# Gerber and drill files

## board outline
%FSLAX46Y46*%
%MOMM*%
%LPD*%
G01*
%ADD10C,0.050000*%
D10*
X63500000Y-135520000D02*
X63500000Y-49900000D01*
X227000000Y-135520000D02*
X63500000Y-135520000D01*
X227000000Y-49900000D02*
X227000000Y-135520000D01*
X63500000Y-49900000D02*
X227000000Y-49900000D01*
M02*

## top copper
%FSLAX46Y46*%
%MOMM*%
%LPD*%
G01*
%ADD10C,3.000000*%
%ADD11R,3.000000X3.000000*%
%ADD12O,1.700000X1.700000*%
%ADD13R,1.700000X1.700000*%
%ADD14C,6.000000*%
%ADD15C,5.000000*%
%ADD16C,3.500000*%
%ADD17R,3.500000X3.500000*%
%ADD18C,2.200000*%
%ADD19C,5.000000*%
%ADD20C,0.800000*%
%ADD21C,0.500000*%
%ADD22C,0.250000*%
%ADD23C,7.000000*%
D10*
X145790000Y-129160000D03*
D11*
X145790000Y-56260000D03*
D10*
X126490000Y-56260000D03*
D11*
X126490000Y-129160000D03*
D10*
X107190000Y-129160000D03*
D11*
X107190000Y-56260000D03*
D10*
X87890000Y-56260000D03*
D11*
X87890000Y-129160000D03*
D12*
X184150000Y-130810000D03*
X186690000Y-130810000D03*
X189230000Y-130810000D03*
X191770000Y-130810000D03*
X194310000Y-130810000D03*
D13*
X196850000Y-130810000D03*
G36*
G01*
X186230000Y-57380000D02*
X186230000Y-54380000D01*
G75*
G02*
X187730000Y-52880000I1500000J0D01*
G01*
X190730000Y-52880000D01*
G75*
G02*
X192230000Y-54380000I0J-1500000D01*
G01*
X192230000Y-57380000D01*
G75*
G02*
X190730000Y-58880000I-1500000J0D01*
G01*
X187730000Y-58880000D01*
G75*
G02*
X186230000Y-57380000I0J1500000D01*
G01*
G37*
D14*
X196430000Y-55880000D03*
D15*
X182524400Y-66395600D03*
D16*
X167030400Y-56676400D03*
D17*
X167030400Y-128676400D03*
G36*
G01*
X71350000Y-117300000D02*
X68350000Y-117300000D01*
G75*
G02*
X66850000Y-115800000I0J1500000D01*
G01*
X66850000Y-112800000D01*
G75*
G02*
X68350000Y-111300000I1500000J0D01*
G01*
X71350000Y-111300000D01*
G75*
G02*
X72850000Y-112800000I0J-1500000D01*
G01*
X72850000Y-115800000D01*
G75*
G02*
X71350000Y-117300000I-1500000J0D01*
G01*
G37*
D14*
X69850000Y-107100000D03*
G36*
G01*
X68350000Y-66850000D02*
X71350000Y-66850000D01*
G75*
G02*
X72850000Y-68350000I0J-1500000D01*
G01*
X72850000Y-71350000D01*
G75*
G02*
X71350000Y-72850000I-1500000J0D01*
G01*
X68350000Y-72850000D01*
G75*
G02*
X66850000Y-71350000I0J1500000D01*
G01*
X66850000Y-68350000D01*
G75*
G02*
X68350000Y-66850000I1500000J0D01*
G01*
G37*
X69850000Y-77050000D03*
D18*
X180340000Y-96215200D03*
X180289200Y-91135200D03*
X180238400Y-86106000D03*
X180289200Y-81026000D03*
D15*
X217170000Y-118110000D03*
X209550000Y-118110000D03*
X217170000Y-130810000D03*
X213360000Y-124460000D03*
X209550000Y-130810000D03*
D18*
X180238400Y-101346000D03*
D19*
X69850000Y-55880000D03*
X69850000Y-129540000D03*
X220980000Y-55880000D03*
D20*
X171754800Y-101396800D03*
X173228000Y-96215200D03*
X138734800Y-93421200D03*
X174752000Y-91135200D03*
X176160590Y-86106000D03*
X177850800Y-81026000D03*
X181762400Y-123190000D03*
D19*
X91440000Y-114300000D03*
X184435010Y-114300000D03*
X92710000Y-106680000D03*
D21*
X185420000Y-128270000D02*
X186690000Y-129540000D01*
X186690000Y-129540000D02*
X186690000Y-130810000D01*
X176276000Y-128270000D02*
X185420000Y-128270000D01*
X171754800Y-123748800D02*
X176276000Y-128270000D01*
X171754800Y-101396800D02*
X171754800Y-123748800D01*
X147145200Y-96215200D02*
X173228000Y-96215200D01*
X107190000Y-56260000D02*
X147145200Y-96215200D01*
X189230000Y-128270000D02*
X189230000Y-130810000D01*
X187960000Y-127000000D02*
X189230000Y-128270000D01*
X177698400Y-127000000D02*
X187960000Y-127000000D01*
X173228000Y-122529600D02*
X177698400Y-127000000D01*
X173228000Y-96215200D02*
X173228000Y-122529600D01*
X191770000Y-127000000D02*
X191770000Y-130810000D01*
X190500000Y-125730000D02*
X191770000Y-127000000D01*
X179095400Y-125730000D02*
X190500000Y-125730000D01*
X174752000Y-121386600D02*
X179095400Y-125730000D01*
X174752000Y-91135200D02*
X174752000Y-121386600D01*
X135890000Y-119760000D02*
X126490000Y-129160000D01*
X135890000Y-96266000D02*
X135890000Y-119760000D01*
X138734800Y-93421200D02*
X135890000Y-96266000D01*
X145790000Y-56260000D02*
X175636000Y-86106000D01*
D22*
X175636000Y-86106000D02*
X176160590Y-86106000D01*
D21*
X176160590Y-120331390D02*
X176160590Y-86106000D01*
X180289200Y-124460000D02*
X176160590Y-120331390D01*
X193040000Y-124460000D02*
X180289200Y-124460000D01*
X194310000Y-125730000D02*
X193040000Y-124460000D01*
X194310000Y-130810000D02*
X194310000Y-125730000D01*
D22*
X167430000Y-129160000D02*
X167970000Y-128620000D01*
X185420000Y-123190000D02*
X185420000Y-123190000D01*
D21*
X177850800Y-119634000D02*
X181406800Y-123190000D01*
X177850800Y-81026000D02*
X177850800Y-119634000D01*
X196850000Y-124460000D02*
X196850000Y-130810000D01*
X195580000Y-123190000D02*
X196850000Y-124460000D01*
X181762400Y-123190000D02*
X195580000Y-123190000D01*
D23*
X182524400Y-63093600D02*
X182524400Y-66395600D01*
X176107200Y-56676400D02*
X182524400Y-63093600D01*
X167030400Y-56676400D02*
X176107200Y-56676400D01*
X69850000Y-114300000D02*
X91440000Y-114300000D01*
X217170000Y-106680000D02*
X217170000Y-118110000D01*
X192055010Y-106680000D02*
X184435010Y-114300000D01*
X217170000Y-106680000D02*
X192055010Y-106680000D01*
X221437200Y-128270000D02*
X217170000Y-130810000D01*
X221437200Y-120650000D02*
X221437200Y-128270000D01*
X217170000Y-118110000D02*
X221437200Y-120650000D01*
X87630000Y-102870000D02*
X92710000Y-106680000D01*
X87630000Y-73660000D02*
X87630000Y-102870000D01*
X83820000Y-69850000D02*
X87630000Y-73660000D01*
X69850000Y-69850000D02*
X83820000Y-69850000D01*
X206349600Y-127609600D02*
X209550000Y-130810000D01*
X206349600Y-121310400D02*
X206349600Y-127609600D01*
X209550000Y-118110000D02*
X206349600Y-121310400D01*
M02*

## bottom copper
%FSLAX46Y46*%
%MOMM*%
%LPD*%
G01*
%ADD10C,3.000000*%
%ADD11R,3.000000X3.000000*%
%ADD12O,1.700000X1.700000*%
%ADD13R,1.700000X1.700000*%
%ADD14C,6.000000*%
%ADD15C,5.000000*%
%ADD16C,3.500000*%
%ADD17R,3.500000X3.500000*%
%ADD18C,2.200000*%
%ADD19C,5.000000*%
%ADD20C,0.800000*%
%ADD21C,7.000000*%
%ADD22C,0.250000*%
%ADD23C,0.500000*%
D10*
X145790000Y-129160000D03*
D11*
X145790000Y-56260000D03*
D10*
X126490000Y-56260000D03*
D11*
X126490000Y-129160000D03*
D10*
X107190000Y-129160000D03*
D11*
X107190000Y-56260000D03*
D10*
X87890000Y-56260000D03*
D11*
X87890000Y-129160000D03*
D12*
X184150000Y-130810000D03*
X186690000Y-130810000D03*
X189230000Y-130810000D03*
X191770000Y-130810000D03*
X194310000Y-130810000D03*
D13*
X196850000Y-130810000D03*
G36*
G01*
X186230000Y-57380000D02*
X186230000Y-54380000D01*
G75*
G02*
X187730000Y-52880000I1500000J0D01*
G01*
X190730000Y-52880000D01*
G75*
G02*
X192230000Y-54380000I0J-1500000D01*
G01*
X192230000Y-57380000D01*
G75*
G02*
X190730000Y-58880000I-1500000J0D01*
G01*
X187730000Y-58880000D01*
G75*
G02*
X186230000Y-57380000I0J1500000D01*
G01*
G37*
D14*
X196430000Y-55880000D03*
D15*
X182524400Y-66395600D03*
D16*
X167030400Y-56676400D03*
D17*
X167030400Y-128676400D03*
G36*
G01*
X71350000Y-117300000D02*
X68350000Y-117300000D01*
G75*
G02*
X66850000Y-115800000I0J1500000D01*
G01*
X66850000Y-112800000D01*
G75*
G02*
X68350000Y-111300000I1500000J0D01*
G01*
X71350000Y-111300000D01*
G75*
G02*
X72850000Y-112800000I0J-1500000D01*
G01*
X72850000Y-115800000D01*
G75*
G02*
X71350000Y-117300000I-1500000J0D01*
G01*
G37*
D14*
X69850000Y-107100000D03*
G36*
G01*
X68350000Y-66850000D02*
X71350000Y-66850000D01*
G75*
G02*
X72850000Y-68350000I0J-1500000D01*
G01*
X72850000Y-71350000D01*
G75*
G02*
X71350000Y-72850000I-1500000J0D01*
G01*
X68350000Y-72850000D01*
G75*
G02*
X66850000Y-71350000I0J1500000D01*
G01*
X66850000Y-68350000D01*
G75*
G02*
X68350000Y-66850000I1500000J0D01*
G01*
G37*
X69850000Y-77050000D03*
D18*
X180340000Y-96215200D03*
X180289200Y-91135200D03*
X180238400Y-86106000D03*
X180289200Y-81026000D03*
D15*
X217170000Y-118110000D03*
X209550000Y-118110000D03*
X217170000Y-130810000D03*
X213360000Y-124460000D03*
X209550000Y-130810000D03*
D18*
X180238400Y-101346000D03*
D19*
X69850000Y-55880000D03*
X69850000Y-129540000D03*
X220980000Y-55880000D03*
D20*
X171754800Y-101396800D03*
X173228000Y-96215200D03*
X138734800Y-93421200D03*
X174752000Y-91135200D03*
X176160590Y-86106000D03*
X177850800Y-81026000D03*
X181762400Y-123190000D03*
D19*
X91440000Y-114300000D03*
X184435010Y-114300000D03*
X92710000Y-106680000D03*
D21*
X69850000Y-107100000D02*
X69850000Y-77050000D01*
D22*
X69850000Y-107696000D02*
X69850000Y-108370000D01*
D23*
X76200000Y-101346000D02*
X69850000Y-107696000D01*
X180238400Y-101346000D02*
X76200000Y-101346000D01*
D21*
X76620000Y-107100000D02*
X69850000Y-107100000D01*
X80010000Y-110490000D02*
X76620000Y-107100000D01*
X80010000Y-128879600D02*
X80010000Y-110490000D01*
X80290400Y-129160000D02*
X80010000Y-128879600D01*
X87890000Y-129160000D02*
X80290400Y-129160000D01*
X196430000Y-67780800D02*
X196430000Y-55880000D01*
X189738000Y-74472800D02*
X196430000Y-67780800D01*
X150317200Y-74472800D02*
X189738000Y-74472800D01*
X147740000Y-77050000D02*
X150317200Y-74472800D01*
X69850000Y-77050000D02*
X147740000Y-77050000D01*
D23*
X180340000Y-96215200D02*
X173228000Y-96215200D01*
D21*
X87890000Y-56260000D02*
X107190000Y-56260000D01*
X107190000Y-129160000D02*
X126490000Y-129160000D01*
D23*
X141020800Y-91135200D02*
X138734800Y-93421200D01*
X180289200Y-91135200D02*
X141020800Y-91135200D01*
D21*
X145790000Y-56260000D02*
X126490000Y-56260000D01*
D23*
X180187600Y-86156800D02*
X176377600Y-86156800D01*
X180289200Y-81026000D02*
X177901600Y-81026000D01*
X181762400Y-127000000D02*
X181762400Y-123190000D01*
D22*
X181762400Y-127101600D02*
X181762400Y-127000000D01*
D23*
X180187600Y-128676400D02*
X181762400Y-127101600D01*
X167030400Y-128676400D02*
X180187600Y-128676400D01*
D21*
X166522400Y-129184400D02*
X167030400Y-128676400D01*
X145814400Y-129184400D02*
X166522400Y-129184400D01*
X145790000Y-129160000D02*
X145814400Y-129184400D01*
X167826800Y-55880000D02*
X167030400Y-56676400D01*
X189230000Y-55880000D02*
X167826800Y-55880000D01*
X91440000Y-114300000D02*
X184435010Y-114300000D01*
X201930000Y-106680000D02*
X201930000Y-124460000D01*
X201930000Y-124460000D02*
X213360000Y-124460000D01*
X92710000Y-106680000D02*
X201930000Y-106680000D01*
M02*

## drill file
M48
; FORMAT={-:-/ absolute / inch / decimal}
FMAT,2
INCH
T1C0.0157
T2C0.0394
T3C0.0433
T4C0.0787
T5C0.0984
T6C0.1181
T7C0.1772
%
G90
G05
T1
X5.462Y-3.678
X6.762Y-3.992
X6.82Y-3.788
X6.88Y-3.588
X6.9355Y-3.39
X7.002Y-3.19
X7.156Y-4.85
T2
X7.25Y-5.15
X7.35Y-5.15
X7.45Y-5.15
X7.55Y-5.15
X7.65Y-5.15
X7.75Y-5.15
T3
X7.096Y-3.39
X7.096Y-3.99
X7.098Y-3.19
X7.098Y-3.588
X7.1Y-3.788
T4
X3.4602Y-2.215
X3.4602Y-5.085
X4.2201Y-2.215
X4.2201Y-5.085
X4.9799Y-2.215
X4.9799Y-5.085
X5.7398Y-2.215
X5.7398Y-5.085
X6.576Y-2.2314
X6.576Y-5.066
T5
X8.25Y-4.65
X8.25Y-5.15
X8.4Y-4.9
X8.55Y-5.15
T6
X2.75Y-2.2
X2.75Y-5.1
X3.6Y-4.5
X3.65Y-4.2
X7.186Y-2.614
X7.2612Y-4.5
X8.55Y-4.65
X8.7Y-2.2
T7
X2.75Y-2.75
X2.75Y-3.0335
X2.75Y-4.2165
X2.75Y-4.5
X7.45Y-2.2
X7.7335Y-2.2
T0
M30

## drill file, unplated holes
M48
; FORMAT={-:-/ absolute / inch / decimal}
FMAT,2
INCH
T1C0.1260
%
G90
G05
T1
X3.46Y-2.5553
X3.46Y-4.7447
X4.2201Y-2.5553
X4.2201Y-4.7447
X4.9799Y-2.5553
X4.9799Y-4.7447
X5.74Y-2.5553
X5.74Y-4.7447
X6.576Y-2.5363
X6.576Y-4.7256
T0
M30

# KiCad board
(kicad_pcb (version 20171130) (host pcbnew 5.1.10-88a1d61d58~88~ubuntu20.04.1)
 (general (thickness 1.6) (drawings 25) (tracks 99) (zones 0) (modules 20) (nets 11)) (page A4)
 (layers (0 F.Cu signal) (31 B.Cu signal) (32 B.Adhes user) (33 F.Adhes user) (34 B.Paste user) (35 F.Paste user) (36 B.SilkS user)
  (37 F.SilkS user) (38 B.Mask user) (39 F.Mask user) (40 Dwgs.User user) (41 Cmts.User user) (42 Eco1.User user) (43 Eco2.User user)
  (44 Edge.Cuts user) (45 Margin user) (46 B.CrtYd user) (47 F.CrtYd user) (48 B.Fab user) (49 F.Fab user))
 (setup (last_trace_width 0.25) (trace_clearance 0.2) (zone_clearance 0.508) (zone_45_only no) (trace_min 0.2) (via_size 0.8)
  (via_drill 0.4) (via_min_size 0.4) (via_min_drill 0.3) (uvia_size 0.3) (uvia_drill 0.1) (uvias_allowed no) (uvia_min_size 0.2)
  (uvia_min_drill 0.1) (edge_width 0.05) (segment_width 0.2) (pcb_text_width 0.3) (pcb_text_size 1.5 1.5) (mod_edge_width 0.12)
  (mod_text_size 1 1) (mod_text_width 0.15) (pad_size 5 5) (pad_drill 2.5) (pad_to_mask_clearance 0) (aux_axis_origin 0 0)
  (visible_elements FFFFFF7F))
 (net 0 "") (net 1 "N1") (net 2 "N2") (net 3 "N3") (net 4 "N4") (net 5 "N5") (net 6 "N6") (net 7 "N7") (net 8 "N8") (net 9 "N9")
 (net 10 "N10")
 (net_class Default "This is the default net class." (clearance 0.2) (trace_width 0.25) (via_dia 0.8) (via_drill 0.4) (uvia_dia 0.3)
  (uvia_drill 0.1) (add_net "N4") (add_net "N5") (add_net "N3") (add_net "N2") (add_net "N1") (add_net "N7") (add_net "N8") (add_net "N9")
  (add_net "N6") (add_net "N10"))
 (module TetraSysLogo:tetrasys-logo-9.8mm (layer B.Cu) (at 107.2388 90.932)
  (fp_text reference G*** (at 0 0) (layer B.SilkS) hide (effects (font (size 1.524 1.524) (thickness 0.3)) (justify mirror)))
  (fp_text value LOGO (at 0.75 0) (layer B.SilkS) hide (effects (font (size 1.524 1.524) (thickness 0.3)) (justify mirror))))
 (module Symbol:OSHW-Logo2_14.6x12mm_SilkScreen (layer B.Cu) (at 206.9084 93.5736)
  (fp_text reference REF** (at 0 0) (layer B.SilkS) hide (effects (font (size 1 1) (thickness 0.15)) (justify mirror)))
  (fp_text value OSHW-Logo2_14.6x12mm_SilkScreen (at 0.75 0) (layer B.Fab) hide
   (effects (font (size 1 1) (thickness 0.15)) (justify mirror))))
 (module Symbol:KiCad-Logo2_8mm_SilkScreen (layer B.Cu) (at 207.3148 78.3336)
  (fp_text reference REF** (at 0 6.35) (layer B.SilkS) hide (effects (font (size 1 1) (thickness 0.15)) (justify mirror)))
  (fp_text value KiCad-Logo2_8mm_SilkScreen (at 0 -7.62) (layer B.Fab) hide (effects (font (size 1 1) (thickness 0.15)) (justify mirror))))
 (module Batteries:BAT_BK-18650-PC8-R (layer F.Cu) (at 116.84 92.71 90)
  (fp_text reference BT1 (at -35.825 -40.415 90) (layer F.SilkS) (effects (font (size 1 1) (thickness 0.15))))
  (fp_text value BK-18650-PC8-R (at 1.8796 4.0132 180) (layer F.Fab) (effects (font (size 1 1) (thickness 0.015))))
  (pad "" np_thru_hole circle (at 27.805 28.955 90) (size 3.2 3.2) (drill 3.2) (layers *.Cu *.Mask))
  (pad None np_thru_hole circle (at 27.805 9.65 90) (size 3.2 3.2) (drill 3.2) (layers *.Cu *.Mask))
  (pad None np_thru_hole circle (at 27.805 -28.955 90) (size 3.2 3.2) (drill 3.2) (layers *.Cu *.Mask))
  (pad "" np_thru_hole circle (at 27.805 -9.65 90) (size 3.2 3.2) (drill 3.2) (layers *.Cu *.Mask))
  (pad None np_thru_hole circle (at -27.805 28.955 90) (size 3.2 3.2) (drill 3.2) (layers *.Cu *.Mask))
  (pad "" np_thru_hole circle (at -27.805 9.65 90) (size 3.2 3.2) (drill 3.2) (layers *.Cu *.Mask))
  (pad "" np_thru_hole circle (at -27.805 -28.955 90) (size 3.2 3.2) (drill 3.2) (layers *.Cu *.Mask))
  (pad None np_thru_hole circle (at -27.805 -9.65 90) (size 3.2 3.2) (drill 3.2) (layers *.Cu *.Mask))
  (pad 4 thru_hole circle (at -36.45 28.95 90) (size 3 3) (drill 2) (layers *.Cu *.Mask) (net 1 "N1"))
  (pad 4+ thru_hole rect (at 36.45 28.95 90) (size 3 3) (drill 2) (layers *.Cu *.Mask) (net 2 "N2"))
  (pad 3 thru_hole circle (at 36.45 9.65 90) (size 3 3) (drill 2) (layers *.Cu *.Mask) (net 2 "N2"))
  (pad 3+ thru_hole rect (at -36.45 9.65 90) (size 3 3) (drill 2) (layers *.Cu *.Mask) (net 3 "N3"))
  (pad 2 thru_hole circle (at -36.45 -9.65 90) (size 3 3) (drill 2) (layers *.Cu *.Mask) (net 3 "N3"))
  (pad 2+ thru_hole rect (at 36.45 -9.65 90) (size 3 3) (drill 2) (layers *.Cu *.Mask) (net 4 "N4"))
  (pad 1 thru_hole circle (at 36.45 -28.95 90) (size 3 3) (drill 2) (layers *.Cu *.Mask) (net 4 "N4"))
  (pad 1+ thru_hole rect (at -36.45 -28.95 90) (size 3 3) (drill 2) (layers *.Cu *.Mask) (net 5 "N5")))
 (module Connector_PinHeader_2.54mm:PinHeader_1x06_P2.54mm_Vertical (layer F.Cu) (at 196.85 130.81 270)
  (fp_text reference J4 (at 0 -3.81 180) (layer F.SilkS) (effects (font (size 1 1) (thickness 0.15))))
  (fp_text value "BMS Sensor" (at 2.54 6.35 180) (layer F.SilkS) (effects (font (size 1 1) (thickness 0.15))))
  (pad 6 thru_hole oval (at 0 12.7 270) (size 1.7 1.7) (drill 1) (layers *.Cu *.Mask) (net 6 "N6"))
  (pad 5 thru_hole oval (at 0 10.16 270) (size 1.7 1.7) (drill 1) (layers *.Cu *.Mask) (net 5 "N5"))
  (pad 4 thru_hole oval (at 0 7.62 270) (size 1.7 1.7) (drill 1) (layers *.Cu *.Mask) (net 4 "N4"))
  (pad 3 thru_hole oval (at 0 5.08 270) (size 1.7 1.7) (drill 1) (layers *.Cu *.Mask) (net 3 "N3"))
  (pad 2 thru_hole oval (at 0 2.54 270) (size 1.7 1.7) (drill 1) (layers *.Cu *.Mask) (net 2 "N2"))
  (pad 1 thru_hole rect (at 0 0 270) (size 1.7 1.7) (drill 1) (layers *.Cu *.Mask) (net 1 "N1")))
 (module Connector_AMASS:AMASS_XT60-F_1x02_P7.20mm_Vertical (layer F.Cu) (at 189.23 55.88)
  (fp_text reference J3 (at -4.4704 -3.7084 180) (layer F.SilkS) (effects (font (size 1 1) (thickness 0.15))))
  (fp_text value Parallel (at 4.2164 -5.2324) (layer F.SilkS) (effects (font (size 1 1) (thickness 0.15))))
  (pad 1 thru_hole roundrect (at 0 0) (size 6 6) (drill 4.5) (layers *.Cu *.Mask) (roundrect_rratio 0.25) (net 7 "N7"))
  (pad 2 thru_hole circle (at 7.2 0) (size 6 6) (drill 4.5) (layers *.Cu *.Mask) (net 5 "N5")))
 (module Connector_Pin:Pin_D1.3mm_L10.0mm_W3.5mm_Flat (layer F.Cu) (at 182.5244 66.3956)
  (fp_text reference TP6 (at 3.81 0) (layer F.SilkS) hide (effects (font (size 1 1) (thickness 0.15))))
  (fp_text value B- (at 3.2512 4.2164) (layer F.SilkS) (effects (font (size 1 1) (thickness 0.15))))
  (pad 1 thru_hole circle (at 0 0) (size 5 5) (drill 3) (layers *.Cu *.Mask) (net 7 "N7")))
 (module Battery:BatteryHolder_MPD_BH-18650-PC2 (layer F.Cu) (at 167.0304 128.6764 90)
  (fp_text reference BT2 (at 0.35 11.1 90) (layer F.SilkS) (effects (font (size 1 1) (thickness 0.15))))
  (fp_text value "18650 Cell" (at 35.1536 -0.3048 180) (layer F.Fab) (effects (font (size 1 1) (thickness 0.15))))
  (pad 2 thru_hole circle (at 72 0 90) (size 3.5 3.5) (drill 2) (layers *.Cu *.Mask) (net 7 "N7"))
  (pad 1 thru_hole rect (at 0 0 90) (size 3.5 3.5) (drill 2) (layers *.Cu *.Mask) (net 1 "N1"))
  (pad "" np_thru_hole circle (at 8.645 0 90) (size 3.2 3.2) (drill 3.2) (layers *.Cu *.Mask))
  (pad "" np_thru_hole circle (at 64.255 0 90) (size 3.2 3.2) (drill 3.2) (layers *.Cu *.Mask)))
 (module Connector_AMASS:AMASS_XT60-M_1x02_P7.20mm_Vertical (layer F.Cu) (at 69.85 114.3 90)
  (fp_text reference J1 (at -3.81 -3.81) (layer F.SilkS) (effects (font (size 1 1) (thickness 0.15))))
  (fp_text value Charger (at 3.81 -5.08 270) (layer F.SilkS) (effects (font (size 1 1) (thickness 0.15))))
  (pad 1 thru_hole roundrect (at 0 0 90) (size 6 6) (drill 4.5) (layers *.Cu *.Mask) (roundrect_rratio 0.25) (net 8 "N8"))
  (pad 2 thru_hole circle (at 7.2 0 90) (size 6 6) (drill 4.5) (layers *.Cu *.Mask) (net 5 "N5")))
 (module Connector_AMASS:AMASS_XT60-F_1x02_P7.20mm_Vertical (layer F.Cu) (at 69.85 69.85 270)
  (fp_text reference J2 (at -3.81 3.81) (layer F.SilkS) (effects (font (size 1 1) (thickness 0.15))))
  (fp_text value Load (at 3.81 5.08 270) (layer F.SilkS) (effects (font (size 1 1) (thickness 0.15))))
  (pad 1 thru_hole roundrect (at 0 0 270) (size 6 6) (drill 4.5) (layers *.Cu *.Mask) (roundrect_rratio 0.25) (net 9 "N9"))
  (pad 2 thru_hole circle (at 7.2 0 270) (size 6 6) (drill 4.5) (layers *.Cu *.Mask) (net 5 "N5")))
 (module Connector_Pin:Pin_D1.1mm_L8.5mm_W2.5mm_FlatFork (layer F.Cu) (at 180.34 96.2152)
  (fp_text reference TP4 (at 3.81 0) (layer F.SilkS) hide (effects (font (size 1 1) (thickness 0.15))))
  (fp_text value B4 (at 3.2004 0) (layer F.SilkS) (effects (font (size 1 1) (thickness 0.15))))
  (pad 1 thru_hole circle (at 0 0) (size 2.2 2.2) (drill 1.1) (layers *.Cu *.Mask) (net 4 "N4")))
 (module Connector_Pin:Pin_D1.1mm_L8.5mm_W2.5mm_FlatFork (layer F.Cu) (at 180.2892 91.1352)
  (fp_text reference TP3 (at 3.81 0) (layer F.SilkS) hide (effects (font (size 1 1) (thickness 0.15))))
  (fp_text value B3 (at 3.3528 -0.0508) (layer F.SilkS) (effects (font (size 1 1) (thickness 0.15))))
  (pad 1 thru_hole circle (at 0 0) (size 2.2 2.2) (drill 1.1) (layers *.Cu *.Mask) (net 3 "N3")))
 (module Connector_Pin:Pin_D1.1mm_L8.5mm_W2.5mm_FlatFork (layer F.Cu) (at 180.2384 86.106)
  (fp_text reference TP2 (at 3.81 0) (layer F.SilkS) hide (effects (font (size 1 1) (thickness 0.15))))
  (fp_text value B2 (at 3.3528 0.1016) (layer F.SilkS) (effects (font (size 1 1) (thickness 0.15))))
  (pad 1 thru_hole circle (at 0 0) (size 2.2 2.2) (drill 1.1) (layers *.Cu *.Mask) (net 2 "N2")))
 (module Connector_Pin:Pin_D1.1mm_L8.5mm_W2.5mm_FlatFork (layer F.Cu) (at 180.2892 81.026)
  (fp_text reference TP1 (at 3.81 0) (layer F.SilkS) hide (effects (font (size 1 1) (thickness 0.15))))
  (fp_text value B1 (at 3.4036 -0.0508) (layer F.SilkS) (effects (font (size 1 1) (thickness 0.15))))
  (pad 1 thru_hole circle (at 0 0) (size 2.2 2.2) (drill 1.1) (layers *.Cu *.Mask) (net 1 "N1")))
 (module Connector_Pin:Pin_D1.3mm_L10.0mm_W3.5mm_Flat (layer F.Cu) (at 217.17 118.11 90)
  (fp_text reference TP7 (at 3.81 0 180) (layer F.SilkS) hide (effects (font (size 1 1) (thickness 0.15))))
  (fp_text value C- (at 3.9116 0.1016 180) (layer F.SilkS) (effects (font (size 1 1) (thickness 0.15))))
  (pad 1 thru_hole circle (at 0 0 90) (size 5 5) (drill 3) (layers *.Cu *.Mask) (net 8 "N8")))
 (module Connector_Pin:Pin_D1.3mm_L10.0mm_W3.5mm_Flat (layer F.Cu) (at 209.55 118.11 90)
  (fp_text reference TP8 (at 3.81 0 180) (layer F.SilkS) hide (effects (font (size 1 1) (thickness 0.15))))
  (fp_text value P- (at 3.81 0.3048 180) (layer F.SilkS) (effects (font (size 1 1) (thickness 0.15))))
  (pad 1 thru_hole circle (at 0 0 90) (size 5 5) (drill 2.5) (layers *.Cu *.Mask) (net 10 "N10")))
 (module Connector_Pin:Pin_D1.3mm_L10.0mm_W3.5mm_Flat (layer F.Cu) (at 217.17 130.81 90)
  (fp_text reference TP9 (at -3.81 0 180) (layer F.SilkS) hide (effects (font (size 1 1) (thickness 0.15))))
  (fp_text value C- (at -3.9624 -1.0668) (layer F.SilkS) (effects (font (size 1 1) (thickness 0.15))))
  (pad 1 thru_hole circle (at 0 0 90) (size 5 5) (drill 2.5) (layers *.Cu *.Mask) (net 8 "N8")))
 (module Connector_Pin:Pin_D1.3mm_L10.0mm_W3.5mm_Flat (layer F.Cu) (at 213.36 124.46 90)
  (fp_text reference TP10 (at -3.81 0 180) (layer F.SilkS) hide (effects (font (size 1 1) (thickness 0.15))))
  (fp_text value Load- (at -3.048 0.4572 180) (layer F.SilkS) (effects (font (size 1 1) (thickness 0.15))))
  (pad 1 thru_hole circle (at 0 0 90) (size 5 5) (drill 2.5) (layers *.Cu *.Mask) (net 9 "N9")))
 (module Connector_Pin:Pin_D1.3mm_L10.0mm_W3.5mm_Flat (layer F.Cu) (at 209.55 130.81 90)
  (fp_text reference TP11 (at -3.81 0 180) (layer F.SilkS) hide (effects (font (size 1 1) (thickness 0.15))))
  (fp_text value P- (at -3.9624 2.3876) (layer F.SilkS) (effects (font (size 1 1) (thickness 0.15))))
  (pad 1 thru_hole circle (at 0 0 90) (size 5 5) (drill 2.5) (layers *.Cu *.Mask) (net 10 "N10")))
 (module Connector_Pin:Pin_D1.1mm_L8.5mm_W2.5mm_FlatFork (layer F.Cu) (at 180.2384 101.346)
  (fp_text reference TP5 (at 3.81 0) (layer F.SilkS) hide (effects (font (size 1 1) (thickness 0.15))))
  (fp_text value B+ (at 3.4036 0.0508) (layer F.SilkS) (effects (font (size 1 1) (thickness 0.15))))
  (pad 1 thru_hole circle (at 0 0) (size 2.2 2.2) (drill 1.1) (layers *.Cu *.Mask) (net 5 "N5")))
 (gr_line (start 63.5 135.52) (end 63.5 49.9) (layer Edge.Cuts) (width 0.05))
 (gr_line (start 227 135.52) (end 63.5 135.52) (layer Edge.Cuts) (width 0.05))
 (gr_line (start 227 49.9) (end 227 135.52) (layer Edge.Cuts) (width 0.05))
 (gr_line (start 63.5 49.9) (end 227 49.9) (layer Edge.Cuts) (width 0.05))
 (via (at 69.85 55.88) (size 5) (drill 3) (layers F.Cu B.Cu) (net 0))
 (via (at 69.85 129.54) (size 5) (drill 3) (layers F.Cu B.Cu) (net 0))
 (via (at 220.98 55.88) (size 5) (drill 3) (layers F.Cu B.Cu) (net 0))
 (via (at 171.7548 101.3968) (size 0.8) (drill 0.4) (layers F.Cu B.Cu) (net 5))
 (segment (start 69.85 107.1) (end 69.85 77.05) (width 7) (layer B.Cu) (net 5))
 (segment (start 69.85 107.696) (end 69.85 108.37) (width 0.25) (layer B.Cu) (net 5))
 (segment (start 76.2 101.346) (end 69.85 107.696) (width 0.5) (layer B.Cu) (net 5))
 (segment (start 180.2384 101.346) (end 76.2 101.346) (width 0.5) (layer B.Cu) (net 5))
 (segment (start 185.42 128.27) (end 186.69 129.54) (width 0.5) (layer F.Cu) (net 5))
 (segment (start 186.69 129.54) (end 186.69 130.81) (width 0.5) (layer F.Cu) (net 5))
 (segment (start 176.276 128.27) (end 185.42 128.27) (width 0.5) (layer F.Cu) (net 5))
 (segment (start 171.7548 123.7488) (end 176.276 128.27) (width 0.5) (layer F.Cu) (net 5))
 (segment (start 171.7548 101.3968) (end 171.7548 123.7488) (width 0.5) (layer F.Cu) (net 5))
 (segment (start 76.62 107.1) (end 69.85 107.1) (width 7) (layer B.Cu) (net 5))
 (segment (start 80.01 110.49) (end 76.62 107.1) (width 7) (layer B.Cu) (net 5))
 (segment (start 80.01 128.8796) (end 80.01 110.49) (width 7) (layer B.Cu) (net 5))
 (segment (start 80.2904 129.16) (end 80.01 128.8796) (width 7) (layer B.Cu) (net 5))
 (segment (start 87.89 129.16) (end 80.2904 129.16) (width 7) (layer B.Cu) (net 5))
 (segment (start 196.43 67.7808) (end 196.43 55.88) (width 7) (layer B.Cu) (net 5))
 (segment (start 189.738 74.4728) (end 196.43 67.7808) (width 7) (layer B.Cu) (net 5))
 (segment (start 150.3172 74.4728) (end 189.738 74.4728) (width 7) (layer B.Cu) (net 5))
 (segment (start 147.74 77.05) (end 150.3172 74.4728) (width 7) (layer B.Cu) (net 5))
 (segment (start 69.85 77.05) (end 147.74 77.05) (width 7) (layer B.Cu) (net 5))
 (via (at 173.228 96.2152) (size 0.8) (drill 0.4) (layers F.Cu B.Cu) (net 4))
 (segment (start 180.34 96.2152) (end 173.228 96.2152) (width 0.5) (layer B.Cu) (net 4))
 (segment (start 147.1452 96.2152) (end 173.228 96.2152) (width 0.5) (layer F.Cu) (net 4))
 (segment (start 107.19 56.26) (end 147.1452 96.2152) (width 0.5) (layer F.Cu) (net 4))
 (segment (start 189.23 128.27) (end 189.23 130.81) (width 0.5) (layer F.Cu) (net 4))
 (segment (start 187.96 127) (end 189.23 128.27) (width 0.5) (layer F.Cu) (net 4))
 (segment (start 177.6984 127) (end 187.96 127) (width 0.5) (layer F.Cu) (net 4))
 (segment (start 173.228 122.5296) (end 177.6984 127) (width 0.5) (layer F.Cu) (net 4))
 (segment (start 173.228 96.2152) (end 173.228 122.5296) (width 0.5) (layer F.Cu) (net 4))
 (segment (start 87.89 56.26) (end 107.19 56.26) (width 7) (layer B.Cu) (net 4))
 (via (at 138.7348 93.4212) (size 0.8) (drill 0.4) (layers F.Cu B.Cu) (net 3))
 (segment (start 107.19 129.16) (end 126.49 129.16) (width 7) (layer B.Cu) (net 3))
 (via (at 174.752 91.1352) (size 0.8) (drill 0.4) (layers F.Cu B.Cu) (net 3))
 (segment (start 191.77 127) (end 191.77 130.81) (width 0.5) (layer F.Cu) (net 3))
 (segment (start 190.5 125.73) (end 191.77 127) (width 0.5) (layer F.Cu) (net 3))
 (segment (start 179.0954 125.73) (end 190.5 125.73) (width 0.5) (layer F.Cu) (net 3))
 (segment (start 174.752 121.3866) (end 179.0954 125.73) (width 0.5) (layer F.Cu) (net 3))
 (segment (start 174.752 91.1352) (end 174.752 121.3866) (width 0.5) (layer F.Cu) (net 3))
 (segment (start 135.89 119.76) (end 126.49 129.16) (width 0.5) (layer F.Cu) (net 3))
 (segment (start 135.89 96.266) (end 135.89 119.76) (width 0.5) (layer F.Cu) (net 3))
 (segment (start 138.7348 93.4212) (end 135.89 96.266) (width 0.5) (layer F.Cu) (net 3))
 (segment (start 141.0208 91.1352) (end 138.7348 93.4212) (width 0.5) (layer B.Cu) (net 3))
 (segment (start 180.2892 91.1352) (end 141.0208 91.1352) (width 0.5) (layer B.Cu) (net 3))
 (segment (start 145.79 56.26) (end 126.49 56.26) (width 7) (layer B.Cu) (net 2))
 (segment (start 180.1876 86.1568) (end 176.3776 86.1568) (width 0.5) (layer B.Cu) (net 2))
 (via (at 176.16059 86.106) (size 0.8) (drill 0.4) (layers F.Cu B.Cu) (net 2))
 (segment (start 145.79 56.26) (end 175.636 86.106) (width 0.5) (layer F.Cu) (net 2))
 (segment (start 175.636 86.106) (end 176.16059 86.106) (width 0.25) (layer F.Cu) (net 2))
 (segment (start 176.16059 120.33139) (end 176.16059 86.106) (width 0.5) (layer F.Cu) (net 2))
 (segment (start 180.2892 124.46) (end 176.16059 120.33139) (width 0.5) (layer F.Cu) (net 2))
 (segment (start 193.04 124.46) (end 180.2892 124.46) (width 0.5) (layer F.Cu) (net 2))
 (segment (start 194.31 125.73) (end 193.04 124.46) (width 0.5) (layer F.Cu) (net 2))
 (segment (start 194.31 130.81) (end 194.31 125.73) (width 0.5) (layer F.Cu) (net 2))
 (via (at 177.8508 81.026) (size 0.8) (drill 0.4) (layers F.Cu B.Cu) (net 1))
 (segment (start 167.43 129.16) (end 167.97 128.62) (width 0.25) (layer F.Cu) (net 1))
 (segment (start 185.42 123.19) (end 185.42 123.19) (width 0.25) (layer F.Cu) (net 1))
 (via (at 181.7624 123.19) (size 0.8) (drill 0.4) (layers F.Cu B.Cu) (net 1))
 (segment (start 180.2892 81.026) (end 177.9016 81.026) (width 0.5) (layer B.Cu) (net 1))
 (segment (start 177.8508 119.634) (end 181.4068 123.19) (width 0.5) (layer F.Cu) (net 1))
 (segment (start 177.8508 81.026) (end 177.8508 119.634) (width 0.5) (layer F.Cu) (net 1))
 (segment (start 181.7624 127) (end 181.7624 123.19) (width 0.5) (layer B.Cu) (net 1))
 (segment (start 181.7624 127.1016) (end 181.7624 127) (width 0.25) (layer B.Cu) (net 1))
 (segment (start 180.1876 128.6764) (end 181.7624 127.1016) (width 0.5) (layer B.Cu) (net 1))
 (segment (start 167.0304 128.6764) (end 180.1876 128.6764) (width 0.5) (layer B.Cu) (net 1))
 (segment (start 196.85 124.46) (end 196.85 130.81) (width 0.5) (layer F.Cu) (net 1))
 (segment (start 195.58 123.19) (end 196.85 124.46) (width 0.5) (layer F.Cu) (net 1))
 (segment (start 181.7624 123.19) (end 195.58 123.19) (width 0.5) (layer F.Cu) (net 1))
 (segment (start 166.5224 129.1844) (end 167.0304 128.6764) (width 7) (layer B.Cu) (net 1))
 (segment (start 145.8144 129.1844) (end 166.5224 129.1844) (width 7) (layer B.Cu) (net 1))
 (segment (start 145.79 129.16) (end 145.8144 129.1844) (width 7) (layer B.Cu) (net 1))
 (segment (start 167.8268 55.88) (end 167.0304 56.6764) (width 7) (layer B.Cu) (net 7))
 (segment (start 189.23 55.88) (end 167.8268 55.88) (width 7) (layer B.Cu) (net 7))
 (segment (start 182.5244 63.0936) (end 182.5244 66.3956) (width 7) (layer F.Cu) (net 7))
 (segment (start 176.1072 56.6764) (end 182.5244 63.0936) (width 7) (layer F.Cu) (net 7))
 (segment (start 167.0304 56.6764) (end 176.1072 56.6764) (width 7) (layer F.Cu) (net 7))
 (via (at 91.44 114.3) (size 5) (drill 3) (layers F.Cu B.Cu) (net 8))
 (via (at 184.43501 114.3) (size 5) (drill 3) (layers F.Cu B.Cu) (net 8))
 (segment (start 69.85 114.3) (end 91.44 114.3) (width 7) (layer F.Cu) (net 8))
 (segment (start 91.44 114.3) (end 184.43501 114.3) (width 7) (layer B.Cu) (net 8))
 (segment (start 217.17 106.68) (end 217.17 118.11) (width 7) (layer F.Cu) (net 8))
 (segment (start 192.05501 106.68) (end 184.43501 114.3) (width 7) (layer F.Cu) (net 8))
 (segment (start 217.17 106.68) (end 192.05501 106.68) (width 7) (layer F.Cu) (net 8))
 (segment (start 221.4372 128.27) (end 217.17 130.81) (width 7) (layer F.Cu) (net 8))
 (segment (start 221.4372 120.65) (end 221.4372 128.27) (width 7) (layer F.Cu) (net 8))
 (segment (start 217.17 118.11) (end 221.4372 120.65) (width 7) (layer F.Cu) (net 8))
 (via (at 92.71 106.68) (size 5) (drill 3) (layers F.Cu B.Cu) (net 9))
 (segment (start 87.63 102.87) (end 92.71 106.68) (width 7) (layer F.Cu) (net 9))
 (segment (start 87.63 73.66) (end 87.63 102.87) (width 7) (layer F.Cu) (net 9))
 (segment (start 83.82 69.85) (end 87.63 73.66) (width 7) (layer F.Cu) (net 9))
 (segment (start 69.85 69.85) (end 83.82 69.85) (width 7) (layer F.Cu) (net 9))
 (segment (start 201.93 106.68) (end 201.93 124.46) (width 7) (layer B.Cu) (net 9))
 (segment (start 201.93 124.46) (end 213.36 124.46) (width 7) (layer B.Cu) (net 9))
 (segment (start 92.71 106.68) (end 201.93 106.68) (width 7) (layer B.Cu) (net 9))
 (segment (start 206.3496 127.6096) (end 209.55 130.81) (width 7) (layer F.Cu) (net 10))
 (segment (start 206.3496 121.3104) (end 206.3496 127.6096) (width 7) (layer F.Cu) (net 10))
 (segment (start 209.55 118.11) (end 206.3496 121.3104) (width 7) (layer F.Cu) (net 10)))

